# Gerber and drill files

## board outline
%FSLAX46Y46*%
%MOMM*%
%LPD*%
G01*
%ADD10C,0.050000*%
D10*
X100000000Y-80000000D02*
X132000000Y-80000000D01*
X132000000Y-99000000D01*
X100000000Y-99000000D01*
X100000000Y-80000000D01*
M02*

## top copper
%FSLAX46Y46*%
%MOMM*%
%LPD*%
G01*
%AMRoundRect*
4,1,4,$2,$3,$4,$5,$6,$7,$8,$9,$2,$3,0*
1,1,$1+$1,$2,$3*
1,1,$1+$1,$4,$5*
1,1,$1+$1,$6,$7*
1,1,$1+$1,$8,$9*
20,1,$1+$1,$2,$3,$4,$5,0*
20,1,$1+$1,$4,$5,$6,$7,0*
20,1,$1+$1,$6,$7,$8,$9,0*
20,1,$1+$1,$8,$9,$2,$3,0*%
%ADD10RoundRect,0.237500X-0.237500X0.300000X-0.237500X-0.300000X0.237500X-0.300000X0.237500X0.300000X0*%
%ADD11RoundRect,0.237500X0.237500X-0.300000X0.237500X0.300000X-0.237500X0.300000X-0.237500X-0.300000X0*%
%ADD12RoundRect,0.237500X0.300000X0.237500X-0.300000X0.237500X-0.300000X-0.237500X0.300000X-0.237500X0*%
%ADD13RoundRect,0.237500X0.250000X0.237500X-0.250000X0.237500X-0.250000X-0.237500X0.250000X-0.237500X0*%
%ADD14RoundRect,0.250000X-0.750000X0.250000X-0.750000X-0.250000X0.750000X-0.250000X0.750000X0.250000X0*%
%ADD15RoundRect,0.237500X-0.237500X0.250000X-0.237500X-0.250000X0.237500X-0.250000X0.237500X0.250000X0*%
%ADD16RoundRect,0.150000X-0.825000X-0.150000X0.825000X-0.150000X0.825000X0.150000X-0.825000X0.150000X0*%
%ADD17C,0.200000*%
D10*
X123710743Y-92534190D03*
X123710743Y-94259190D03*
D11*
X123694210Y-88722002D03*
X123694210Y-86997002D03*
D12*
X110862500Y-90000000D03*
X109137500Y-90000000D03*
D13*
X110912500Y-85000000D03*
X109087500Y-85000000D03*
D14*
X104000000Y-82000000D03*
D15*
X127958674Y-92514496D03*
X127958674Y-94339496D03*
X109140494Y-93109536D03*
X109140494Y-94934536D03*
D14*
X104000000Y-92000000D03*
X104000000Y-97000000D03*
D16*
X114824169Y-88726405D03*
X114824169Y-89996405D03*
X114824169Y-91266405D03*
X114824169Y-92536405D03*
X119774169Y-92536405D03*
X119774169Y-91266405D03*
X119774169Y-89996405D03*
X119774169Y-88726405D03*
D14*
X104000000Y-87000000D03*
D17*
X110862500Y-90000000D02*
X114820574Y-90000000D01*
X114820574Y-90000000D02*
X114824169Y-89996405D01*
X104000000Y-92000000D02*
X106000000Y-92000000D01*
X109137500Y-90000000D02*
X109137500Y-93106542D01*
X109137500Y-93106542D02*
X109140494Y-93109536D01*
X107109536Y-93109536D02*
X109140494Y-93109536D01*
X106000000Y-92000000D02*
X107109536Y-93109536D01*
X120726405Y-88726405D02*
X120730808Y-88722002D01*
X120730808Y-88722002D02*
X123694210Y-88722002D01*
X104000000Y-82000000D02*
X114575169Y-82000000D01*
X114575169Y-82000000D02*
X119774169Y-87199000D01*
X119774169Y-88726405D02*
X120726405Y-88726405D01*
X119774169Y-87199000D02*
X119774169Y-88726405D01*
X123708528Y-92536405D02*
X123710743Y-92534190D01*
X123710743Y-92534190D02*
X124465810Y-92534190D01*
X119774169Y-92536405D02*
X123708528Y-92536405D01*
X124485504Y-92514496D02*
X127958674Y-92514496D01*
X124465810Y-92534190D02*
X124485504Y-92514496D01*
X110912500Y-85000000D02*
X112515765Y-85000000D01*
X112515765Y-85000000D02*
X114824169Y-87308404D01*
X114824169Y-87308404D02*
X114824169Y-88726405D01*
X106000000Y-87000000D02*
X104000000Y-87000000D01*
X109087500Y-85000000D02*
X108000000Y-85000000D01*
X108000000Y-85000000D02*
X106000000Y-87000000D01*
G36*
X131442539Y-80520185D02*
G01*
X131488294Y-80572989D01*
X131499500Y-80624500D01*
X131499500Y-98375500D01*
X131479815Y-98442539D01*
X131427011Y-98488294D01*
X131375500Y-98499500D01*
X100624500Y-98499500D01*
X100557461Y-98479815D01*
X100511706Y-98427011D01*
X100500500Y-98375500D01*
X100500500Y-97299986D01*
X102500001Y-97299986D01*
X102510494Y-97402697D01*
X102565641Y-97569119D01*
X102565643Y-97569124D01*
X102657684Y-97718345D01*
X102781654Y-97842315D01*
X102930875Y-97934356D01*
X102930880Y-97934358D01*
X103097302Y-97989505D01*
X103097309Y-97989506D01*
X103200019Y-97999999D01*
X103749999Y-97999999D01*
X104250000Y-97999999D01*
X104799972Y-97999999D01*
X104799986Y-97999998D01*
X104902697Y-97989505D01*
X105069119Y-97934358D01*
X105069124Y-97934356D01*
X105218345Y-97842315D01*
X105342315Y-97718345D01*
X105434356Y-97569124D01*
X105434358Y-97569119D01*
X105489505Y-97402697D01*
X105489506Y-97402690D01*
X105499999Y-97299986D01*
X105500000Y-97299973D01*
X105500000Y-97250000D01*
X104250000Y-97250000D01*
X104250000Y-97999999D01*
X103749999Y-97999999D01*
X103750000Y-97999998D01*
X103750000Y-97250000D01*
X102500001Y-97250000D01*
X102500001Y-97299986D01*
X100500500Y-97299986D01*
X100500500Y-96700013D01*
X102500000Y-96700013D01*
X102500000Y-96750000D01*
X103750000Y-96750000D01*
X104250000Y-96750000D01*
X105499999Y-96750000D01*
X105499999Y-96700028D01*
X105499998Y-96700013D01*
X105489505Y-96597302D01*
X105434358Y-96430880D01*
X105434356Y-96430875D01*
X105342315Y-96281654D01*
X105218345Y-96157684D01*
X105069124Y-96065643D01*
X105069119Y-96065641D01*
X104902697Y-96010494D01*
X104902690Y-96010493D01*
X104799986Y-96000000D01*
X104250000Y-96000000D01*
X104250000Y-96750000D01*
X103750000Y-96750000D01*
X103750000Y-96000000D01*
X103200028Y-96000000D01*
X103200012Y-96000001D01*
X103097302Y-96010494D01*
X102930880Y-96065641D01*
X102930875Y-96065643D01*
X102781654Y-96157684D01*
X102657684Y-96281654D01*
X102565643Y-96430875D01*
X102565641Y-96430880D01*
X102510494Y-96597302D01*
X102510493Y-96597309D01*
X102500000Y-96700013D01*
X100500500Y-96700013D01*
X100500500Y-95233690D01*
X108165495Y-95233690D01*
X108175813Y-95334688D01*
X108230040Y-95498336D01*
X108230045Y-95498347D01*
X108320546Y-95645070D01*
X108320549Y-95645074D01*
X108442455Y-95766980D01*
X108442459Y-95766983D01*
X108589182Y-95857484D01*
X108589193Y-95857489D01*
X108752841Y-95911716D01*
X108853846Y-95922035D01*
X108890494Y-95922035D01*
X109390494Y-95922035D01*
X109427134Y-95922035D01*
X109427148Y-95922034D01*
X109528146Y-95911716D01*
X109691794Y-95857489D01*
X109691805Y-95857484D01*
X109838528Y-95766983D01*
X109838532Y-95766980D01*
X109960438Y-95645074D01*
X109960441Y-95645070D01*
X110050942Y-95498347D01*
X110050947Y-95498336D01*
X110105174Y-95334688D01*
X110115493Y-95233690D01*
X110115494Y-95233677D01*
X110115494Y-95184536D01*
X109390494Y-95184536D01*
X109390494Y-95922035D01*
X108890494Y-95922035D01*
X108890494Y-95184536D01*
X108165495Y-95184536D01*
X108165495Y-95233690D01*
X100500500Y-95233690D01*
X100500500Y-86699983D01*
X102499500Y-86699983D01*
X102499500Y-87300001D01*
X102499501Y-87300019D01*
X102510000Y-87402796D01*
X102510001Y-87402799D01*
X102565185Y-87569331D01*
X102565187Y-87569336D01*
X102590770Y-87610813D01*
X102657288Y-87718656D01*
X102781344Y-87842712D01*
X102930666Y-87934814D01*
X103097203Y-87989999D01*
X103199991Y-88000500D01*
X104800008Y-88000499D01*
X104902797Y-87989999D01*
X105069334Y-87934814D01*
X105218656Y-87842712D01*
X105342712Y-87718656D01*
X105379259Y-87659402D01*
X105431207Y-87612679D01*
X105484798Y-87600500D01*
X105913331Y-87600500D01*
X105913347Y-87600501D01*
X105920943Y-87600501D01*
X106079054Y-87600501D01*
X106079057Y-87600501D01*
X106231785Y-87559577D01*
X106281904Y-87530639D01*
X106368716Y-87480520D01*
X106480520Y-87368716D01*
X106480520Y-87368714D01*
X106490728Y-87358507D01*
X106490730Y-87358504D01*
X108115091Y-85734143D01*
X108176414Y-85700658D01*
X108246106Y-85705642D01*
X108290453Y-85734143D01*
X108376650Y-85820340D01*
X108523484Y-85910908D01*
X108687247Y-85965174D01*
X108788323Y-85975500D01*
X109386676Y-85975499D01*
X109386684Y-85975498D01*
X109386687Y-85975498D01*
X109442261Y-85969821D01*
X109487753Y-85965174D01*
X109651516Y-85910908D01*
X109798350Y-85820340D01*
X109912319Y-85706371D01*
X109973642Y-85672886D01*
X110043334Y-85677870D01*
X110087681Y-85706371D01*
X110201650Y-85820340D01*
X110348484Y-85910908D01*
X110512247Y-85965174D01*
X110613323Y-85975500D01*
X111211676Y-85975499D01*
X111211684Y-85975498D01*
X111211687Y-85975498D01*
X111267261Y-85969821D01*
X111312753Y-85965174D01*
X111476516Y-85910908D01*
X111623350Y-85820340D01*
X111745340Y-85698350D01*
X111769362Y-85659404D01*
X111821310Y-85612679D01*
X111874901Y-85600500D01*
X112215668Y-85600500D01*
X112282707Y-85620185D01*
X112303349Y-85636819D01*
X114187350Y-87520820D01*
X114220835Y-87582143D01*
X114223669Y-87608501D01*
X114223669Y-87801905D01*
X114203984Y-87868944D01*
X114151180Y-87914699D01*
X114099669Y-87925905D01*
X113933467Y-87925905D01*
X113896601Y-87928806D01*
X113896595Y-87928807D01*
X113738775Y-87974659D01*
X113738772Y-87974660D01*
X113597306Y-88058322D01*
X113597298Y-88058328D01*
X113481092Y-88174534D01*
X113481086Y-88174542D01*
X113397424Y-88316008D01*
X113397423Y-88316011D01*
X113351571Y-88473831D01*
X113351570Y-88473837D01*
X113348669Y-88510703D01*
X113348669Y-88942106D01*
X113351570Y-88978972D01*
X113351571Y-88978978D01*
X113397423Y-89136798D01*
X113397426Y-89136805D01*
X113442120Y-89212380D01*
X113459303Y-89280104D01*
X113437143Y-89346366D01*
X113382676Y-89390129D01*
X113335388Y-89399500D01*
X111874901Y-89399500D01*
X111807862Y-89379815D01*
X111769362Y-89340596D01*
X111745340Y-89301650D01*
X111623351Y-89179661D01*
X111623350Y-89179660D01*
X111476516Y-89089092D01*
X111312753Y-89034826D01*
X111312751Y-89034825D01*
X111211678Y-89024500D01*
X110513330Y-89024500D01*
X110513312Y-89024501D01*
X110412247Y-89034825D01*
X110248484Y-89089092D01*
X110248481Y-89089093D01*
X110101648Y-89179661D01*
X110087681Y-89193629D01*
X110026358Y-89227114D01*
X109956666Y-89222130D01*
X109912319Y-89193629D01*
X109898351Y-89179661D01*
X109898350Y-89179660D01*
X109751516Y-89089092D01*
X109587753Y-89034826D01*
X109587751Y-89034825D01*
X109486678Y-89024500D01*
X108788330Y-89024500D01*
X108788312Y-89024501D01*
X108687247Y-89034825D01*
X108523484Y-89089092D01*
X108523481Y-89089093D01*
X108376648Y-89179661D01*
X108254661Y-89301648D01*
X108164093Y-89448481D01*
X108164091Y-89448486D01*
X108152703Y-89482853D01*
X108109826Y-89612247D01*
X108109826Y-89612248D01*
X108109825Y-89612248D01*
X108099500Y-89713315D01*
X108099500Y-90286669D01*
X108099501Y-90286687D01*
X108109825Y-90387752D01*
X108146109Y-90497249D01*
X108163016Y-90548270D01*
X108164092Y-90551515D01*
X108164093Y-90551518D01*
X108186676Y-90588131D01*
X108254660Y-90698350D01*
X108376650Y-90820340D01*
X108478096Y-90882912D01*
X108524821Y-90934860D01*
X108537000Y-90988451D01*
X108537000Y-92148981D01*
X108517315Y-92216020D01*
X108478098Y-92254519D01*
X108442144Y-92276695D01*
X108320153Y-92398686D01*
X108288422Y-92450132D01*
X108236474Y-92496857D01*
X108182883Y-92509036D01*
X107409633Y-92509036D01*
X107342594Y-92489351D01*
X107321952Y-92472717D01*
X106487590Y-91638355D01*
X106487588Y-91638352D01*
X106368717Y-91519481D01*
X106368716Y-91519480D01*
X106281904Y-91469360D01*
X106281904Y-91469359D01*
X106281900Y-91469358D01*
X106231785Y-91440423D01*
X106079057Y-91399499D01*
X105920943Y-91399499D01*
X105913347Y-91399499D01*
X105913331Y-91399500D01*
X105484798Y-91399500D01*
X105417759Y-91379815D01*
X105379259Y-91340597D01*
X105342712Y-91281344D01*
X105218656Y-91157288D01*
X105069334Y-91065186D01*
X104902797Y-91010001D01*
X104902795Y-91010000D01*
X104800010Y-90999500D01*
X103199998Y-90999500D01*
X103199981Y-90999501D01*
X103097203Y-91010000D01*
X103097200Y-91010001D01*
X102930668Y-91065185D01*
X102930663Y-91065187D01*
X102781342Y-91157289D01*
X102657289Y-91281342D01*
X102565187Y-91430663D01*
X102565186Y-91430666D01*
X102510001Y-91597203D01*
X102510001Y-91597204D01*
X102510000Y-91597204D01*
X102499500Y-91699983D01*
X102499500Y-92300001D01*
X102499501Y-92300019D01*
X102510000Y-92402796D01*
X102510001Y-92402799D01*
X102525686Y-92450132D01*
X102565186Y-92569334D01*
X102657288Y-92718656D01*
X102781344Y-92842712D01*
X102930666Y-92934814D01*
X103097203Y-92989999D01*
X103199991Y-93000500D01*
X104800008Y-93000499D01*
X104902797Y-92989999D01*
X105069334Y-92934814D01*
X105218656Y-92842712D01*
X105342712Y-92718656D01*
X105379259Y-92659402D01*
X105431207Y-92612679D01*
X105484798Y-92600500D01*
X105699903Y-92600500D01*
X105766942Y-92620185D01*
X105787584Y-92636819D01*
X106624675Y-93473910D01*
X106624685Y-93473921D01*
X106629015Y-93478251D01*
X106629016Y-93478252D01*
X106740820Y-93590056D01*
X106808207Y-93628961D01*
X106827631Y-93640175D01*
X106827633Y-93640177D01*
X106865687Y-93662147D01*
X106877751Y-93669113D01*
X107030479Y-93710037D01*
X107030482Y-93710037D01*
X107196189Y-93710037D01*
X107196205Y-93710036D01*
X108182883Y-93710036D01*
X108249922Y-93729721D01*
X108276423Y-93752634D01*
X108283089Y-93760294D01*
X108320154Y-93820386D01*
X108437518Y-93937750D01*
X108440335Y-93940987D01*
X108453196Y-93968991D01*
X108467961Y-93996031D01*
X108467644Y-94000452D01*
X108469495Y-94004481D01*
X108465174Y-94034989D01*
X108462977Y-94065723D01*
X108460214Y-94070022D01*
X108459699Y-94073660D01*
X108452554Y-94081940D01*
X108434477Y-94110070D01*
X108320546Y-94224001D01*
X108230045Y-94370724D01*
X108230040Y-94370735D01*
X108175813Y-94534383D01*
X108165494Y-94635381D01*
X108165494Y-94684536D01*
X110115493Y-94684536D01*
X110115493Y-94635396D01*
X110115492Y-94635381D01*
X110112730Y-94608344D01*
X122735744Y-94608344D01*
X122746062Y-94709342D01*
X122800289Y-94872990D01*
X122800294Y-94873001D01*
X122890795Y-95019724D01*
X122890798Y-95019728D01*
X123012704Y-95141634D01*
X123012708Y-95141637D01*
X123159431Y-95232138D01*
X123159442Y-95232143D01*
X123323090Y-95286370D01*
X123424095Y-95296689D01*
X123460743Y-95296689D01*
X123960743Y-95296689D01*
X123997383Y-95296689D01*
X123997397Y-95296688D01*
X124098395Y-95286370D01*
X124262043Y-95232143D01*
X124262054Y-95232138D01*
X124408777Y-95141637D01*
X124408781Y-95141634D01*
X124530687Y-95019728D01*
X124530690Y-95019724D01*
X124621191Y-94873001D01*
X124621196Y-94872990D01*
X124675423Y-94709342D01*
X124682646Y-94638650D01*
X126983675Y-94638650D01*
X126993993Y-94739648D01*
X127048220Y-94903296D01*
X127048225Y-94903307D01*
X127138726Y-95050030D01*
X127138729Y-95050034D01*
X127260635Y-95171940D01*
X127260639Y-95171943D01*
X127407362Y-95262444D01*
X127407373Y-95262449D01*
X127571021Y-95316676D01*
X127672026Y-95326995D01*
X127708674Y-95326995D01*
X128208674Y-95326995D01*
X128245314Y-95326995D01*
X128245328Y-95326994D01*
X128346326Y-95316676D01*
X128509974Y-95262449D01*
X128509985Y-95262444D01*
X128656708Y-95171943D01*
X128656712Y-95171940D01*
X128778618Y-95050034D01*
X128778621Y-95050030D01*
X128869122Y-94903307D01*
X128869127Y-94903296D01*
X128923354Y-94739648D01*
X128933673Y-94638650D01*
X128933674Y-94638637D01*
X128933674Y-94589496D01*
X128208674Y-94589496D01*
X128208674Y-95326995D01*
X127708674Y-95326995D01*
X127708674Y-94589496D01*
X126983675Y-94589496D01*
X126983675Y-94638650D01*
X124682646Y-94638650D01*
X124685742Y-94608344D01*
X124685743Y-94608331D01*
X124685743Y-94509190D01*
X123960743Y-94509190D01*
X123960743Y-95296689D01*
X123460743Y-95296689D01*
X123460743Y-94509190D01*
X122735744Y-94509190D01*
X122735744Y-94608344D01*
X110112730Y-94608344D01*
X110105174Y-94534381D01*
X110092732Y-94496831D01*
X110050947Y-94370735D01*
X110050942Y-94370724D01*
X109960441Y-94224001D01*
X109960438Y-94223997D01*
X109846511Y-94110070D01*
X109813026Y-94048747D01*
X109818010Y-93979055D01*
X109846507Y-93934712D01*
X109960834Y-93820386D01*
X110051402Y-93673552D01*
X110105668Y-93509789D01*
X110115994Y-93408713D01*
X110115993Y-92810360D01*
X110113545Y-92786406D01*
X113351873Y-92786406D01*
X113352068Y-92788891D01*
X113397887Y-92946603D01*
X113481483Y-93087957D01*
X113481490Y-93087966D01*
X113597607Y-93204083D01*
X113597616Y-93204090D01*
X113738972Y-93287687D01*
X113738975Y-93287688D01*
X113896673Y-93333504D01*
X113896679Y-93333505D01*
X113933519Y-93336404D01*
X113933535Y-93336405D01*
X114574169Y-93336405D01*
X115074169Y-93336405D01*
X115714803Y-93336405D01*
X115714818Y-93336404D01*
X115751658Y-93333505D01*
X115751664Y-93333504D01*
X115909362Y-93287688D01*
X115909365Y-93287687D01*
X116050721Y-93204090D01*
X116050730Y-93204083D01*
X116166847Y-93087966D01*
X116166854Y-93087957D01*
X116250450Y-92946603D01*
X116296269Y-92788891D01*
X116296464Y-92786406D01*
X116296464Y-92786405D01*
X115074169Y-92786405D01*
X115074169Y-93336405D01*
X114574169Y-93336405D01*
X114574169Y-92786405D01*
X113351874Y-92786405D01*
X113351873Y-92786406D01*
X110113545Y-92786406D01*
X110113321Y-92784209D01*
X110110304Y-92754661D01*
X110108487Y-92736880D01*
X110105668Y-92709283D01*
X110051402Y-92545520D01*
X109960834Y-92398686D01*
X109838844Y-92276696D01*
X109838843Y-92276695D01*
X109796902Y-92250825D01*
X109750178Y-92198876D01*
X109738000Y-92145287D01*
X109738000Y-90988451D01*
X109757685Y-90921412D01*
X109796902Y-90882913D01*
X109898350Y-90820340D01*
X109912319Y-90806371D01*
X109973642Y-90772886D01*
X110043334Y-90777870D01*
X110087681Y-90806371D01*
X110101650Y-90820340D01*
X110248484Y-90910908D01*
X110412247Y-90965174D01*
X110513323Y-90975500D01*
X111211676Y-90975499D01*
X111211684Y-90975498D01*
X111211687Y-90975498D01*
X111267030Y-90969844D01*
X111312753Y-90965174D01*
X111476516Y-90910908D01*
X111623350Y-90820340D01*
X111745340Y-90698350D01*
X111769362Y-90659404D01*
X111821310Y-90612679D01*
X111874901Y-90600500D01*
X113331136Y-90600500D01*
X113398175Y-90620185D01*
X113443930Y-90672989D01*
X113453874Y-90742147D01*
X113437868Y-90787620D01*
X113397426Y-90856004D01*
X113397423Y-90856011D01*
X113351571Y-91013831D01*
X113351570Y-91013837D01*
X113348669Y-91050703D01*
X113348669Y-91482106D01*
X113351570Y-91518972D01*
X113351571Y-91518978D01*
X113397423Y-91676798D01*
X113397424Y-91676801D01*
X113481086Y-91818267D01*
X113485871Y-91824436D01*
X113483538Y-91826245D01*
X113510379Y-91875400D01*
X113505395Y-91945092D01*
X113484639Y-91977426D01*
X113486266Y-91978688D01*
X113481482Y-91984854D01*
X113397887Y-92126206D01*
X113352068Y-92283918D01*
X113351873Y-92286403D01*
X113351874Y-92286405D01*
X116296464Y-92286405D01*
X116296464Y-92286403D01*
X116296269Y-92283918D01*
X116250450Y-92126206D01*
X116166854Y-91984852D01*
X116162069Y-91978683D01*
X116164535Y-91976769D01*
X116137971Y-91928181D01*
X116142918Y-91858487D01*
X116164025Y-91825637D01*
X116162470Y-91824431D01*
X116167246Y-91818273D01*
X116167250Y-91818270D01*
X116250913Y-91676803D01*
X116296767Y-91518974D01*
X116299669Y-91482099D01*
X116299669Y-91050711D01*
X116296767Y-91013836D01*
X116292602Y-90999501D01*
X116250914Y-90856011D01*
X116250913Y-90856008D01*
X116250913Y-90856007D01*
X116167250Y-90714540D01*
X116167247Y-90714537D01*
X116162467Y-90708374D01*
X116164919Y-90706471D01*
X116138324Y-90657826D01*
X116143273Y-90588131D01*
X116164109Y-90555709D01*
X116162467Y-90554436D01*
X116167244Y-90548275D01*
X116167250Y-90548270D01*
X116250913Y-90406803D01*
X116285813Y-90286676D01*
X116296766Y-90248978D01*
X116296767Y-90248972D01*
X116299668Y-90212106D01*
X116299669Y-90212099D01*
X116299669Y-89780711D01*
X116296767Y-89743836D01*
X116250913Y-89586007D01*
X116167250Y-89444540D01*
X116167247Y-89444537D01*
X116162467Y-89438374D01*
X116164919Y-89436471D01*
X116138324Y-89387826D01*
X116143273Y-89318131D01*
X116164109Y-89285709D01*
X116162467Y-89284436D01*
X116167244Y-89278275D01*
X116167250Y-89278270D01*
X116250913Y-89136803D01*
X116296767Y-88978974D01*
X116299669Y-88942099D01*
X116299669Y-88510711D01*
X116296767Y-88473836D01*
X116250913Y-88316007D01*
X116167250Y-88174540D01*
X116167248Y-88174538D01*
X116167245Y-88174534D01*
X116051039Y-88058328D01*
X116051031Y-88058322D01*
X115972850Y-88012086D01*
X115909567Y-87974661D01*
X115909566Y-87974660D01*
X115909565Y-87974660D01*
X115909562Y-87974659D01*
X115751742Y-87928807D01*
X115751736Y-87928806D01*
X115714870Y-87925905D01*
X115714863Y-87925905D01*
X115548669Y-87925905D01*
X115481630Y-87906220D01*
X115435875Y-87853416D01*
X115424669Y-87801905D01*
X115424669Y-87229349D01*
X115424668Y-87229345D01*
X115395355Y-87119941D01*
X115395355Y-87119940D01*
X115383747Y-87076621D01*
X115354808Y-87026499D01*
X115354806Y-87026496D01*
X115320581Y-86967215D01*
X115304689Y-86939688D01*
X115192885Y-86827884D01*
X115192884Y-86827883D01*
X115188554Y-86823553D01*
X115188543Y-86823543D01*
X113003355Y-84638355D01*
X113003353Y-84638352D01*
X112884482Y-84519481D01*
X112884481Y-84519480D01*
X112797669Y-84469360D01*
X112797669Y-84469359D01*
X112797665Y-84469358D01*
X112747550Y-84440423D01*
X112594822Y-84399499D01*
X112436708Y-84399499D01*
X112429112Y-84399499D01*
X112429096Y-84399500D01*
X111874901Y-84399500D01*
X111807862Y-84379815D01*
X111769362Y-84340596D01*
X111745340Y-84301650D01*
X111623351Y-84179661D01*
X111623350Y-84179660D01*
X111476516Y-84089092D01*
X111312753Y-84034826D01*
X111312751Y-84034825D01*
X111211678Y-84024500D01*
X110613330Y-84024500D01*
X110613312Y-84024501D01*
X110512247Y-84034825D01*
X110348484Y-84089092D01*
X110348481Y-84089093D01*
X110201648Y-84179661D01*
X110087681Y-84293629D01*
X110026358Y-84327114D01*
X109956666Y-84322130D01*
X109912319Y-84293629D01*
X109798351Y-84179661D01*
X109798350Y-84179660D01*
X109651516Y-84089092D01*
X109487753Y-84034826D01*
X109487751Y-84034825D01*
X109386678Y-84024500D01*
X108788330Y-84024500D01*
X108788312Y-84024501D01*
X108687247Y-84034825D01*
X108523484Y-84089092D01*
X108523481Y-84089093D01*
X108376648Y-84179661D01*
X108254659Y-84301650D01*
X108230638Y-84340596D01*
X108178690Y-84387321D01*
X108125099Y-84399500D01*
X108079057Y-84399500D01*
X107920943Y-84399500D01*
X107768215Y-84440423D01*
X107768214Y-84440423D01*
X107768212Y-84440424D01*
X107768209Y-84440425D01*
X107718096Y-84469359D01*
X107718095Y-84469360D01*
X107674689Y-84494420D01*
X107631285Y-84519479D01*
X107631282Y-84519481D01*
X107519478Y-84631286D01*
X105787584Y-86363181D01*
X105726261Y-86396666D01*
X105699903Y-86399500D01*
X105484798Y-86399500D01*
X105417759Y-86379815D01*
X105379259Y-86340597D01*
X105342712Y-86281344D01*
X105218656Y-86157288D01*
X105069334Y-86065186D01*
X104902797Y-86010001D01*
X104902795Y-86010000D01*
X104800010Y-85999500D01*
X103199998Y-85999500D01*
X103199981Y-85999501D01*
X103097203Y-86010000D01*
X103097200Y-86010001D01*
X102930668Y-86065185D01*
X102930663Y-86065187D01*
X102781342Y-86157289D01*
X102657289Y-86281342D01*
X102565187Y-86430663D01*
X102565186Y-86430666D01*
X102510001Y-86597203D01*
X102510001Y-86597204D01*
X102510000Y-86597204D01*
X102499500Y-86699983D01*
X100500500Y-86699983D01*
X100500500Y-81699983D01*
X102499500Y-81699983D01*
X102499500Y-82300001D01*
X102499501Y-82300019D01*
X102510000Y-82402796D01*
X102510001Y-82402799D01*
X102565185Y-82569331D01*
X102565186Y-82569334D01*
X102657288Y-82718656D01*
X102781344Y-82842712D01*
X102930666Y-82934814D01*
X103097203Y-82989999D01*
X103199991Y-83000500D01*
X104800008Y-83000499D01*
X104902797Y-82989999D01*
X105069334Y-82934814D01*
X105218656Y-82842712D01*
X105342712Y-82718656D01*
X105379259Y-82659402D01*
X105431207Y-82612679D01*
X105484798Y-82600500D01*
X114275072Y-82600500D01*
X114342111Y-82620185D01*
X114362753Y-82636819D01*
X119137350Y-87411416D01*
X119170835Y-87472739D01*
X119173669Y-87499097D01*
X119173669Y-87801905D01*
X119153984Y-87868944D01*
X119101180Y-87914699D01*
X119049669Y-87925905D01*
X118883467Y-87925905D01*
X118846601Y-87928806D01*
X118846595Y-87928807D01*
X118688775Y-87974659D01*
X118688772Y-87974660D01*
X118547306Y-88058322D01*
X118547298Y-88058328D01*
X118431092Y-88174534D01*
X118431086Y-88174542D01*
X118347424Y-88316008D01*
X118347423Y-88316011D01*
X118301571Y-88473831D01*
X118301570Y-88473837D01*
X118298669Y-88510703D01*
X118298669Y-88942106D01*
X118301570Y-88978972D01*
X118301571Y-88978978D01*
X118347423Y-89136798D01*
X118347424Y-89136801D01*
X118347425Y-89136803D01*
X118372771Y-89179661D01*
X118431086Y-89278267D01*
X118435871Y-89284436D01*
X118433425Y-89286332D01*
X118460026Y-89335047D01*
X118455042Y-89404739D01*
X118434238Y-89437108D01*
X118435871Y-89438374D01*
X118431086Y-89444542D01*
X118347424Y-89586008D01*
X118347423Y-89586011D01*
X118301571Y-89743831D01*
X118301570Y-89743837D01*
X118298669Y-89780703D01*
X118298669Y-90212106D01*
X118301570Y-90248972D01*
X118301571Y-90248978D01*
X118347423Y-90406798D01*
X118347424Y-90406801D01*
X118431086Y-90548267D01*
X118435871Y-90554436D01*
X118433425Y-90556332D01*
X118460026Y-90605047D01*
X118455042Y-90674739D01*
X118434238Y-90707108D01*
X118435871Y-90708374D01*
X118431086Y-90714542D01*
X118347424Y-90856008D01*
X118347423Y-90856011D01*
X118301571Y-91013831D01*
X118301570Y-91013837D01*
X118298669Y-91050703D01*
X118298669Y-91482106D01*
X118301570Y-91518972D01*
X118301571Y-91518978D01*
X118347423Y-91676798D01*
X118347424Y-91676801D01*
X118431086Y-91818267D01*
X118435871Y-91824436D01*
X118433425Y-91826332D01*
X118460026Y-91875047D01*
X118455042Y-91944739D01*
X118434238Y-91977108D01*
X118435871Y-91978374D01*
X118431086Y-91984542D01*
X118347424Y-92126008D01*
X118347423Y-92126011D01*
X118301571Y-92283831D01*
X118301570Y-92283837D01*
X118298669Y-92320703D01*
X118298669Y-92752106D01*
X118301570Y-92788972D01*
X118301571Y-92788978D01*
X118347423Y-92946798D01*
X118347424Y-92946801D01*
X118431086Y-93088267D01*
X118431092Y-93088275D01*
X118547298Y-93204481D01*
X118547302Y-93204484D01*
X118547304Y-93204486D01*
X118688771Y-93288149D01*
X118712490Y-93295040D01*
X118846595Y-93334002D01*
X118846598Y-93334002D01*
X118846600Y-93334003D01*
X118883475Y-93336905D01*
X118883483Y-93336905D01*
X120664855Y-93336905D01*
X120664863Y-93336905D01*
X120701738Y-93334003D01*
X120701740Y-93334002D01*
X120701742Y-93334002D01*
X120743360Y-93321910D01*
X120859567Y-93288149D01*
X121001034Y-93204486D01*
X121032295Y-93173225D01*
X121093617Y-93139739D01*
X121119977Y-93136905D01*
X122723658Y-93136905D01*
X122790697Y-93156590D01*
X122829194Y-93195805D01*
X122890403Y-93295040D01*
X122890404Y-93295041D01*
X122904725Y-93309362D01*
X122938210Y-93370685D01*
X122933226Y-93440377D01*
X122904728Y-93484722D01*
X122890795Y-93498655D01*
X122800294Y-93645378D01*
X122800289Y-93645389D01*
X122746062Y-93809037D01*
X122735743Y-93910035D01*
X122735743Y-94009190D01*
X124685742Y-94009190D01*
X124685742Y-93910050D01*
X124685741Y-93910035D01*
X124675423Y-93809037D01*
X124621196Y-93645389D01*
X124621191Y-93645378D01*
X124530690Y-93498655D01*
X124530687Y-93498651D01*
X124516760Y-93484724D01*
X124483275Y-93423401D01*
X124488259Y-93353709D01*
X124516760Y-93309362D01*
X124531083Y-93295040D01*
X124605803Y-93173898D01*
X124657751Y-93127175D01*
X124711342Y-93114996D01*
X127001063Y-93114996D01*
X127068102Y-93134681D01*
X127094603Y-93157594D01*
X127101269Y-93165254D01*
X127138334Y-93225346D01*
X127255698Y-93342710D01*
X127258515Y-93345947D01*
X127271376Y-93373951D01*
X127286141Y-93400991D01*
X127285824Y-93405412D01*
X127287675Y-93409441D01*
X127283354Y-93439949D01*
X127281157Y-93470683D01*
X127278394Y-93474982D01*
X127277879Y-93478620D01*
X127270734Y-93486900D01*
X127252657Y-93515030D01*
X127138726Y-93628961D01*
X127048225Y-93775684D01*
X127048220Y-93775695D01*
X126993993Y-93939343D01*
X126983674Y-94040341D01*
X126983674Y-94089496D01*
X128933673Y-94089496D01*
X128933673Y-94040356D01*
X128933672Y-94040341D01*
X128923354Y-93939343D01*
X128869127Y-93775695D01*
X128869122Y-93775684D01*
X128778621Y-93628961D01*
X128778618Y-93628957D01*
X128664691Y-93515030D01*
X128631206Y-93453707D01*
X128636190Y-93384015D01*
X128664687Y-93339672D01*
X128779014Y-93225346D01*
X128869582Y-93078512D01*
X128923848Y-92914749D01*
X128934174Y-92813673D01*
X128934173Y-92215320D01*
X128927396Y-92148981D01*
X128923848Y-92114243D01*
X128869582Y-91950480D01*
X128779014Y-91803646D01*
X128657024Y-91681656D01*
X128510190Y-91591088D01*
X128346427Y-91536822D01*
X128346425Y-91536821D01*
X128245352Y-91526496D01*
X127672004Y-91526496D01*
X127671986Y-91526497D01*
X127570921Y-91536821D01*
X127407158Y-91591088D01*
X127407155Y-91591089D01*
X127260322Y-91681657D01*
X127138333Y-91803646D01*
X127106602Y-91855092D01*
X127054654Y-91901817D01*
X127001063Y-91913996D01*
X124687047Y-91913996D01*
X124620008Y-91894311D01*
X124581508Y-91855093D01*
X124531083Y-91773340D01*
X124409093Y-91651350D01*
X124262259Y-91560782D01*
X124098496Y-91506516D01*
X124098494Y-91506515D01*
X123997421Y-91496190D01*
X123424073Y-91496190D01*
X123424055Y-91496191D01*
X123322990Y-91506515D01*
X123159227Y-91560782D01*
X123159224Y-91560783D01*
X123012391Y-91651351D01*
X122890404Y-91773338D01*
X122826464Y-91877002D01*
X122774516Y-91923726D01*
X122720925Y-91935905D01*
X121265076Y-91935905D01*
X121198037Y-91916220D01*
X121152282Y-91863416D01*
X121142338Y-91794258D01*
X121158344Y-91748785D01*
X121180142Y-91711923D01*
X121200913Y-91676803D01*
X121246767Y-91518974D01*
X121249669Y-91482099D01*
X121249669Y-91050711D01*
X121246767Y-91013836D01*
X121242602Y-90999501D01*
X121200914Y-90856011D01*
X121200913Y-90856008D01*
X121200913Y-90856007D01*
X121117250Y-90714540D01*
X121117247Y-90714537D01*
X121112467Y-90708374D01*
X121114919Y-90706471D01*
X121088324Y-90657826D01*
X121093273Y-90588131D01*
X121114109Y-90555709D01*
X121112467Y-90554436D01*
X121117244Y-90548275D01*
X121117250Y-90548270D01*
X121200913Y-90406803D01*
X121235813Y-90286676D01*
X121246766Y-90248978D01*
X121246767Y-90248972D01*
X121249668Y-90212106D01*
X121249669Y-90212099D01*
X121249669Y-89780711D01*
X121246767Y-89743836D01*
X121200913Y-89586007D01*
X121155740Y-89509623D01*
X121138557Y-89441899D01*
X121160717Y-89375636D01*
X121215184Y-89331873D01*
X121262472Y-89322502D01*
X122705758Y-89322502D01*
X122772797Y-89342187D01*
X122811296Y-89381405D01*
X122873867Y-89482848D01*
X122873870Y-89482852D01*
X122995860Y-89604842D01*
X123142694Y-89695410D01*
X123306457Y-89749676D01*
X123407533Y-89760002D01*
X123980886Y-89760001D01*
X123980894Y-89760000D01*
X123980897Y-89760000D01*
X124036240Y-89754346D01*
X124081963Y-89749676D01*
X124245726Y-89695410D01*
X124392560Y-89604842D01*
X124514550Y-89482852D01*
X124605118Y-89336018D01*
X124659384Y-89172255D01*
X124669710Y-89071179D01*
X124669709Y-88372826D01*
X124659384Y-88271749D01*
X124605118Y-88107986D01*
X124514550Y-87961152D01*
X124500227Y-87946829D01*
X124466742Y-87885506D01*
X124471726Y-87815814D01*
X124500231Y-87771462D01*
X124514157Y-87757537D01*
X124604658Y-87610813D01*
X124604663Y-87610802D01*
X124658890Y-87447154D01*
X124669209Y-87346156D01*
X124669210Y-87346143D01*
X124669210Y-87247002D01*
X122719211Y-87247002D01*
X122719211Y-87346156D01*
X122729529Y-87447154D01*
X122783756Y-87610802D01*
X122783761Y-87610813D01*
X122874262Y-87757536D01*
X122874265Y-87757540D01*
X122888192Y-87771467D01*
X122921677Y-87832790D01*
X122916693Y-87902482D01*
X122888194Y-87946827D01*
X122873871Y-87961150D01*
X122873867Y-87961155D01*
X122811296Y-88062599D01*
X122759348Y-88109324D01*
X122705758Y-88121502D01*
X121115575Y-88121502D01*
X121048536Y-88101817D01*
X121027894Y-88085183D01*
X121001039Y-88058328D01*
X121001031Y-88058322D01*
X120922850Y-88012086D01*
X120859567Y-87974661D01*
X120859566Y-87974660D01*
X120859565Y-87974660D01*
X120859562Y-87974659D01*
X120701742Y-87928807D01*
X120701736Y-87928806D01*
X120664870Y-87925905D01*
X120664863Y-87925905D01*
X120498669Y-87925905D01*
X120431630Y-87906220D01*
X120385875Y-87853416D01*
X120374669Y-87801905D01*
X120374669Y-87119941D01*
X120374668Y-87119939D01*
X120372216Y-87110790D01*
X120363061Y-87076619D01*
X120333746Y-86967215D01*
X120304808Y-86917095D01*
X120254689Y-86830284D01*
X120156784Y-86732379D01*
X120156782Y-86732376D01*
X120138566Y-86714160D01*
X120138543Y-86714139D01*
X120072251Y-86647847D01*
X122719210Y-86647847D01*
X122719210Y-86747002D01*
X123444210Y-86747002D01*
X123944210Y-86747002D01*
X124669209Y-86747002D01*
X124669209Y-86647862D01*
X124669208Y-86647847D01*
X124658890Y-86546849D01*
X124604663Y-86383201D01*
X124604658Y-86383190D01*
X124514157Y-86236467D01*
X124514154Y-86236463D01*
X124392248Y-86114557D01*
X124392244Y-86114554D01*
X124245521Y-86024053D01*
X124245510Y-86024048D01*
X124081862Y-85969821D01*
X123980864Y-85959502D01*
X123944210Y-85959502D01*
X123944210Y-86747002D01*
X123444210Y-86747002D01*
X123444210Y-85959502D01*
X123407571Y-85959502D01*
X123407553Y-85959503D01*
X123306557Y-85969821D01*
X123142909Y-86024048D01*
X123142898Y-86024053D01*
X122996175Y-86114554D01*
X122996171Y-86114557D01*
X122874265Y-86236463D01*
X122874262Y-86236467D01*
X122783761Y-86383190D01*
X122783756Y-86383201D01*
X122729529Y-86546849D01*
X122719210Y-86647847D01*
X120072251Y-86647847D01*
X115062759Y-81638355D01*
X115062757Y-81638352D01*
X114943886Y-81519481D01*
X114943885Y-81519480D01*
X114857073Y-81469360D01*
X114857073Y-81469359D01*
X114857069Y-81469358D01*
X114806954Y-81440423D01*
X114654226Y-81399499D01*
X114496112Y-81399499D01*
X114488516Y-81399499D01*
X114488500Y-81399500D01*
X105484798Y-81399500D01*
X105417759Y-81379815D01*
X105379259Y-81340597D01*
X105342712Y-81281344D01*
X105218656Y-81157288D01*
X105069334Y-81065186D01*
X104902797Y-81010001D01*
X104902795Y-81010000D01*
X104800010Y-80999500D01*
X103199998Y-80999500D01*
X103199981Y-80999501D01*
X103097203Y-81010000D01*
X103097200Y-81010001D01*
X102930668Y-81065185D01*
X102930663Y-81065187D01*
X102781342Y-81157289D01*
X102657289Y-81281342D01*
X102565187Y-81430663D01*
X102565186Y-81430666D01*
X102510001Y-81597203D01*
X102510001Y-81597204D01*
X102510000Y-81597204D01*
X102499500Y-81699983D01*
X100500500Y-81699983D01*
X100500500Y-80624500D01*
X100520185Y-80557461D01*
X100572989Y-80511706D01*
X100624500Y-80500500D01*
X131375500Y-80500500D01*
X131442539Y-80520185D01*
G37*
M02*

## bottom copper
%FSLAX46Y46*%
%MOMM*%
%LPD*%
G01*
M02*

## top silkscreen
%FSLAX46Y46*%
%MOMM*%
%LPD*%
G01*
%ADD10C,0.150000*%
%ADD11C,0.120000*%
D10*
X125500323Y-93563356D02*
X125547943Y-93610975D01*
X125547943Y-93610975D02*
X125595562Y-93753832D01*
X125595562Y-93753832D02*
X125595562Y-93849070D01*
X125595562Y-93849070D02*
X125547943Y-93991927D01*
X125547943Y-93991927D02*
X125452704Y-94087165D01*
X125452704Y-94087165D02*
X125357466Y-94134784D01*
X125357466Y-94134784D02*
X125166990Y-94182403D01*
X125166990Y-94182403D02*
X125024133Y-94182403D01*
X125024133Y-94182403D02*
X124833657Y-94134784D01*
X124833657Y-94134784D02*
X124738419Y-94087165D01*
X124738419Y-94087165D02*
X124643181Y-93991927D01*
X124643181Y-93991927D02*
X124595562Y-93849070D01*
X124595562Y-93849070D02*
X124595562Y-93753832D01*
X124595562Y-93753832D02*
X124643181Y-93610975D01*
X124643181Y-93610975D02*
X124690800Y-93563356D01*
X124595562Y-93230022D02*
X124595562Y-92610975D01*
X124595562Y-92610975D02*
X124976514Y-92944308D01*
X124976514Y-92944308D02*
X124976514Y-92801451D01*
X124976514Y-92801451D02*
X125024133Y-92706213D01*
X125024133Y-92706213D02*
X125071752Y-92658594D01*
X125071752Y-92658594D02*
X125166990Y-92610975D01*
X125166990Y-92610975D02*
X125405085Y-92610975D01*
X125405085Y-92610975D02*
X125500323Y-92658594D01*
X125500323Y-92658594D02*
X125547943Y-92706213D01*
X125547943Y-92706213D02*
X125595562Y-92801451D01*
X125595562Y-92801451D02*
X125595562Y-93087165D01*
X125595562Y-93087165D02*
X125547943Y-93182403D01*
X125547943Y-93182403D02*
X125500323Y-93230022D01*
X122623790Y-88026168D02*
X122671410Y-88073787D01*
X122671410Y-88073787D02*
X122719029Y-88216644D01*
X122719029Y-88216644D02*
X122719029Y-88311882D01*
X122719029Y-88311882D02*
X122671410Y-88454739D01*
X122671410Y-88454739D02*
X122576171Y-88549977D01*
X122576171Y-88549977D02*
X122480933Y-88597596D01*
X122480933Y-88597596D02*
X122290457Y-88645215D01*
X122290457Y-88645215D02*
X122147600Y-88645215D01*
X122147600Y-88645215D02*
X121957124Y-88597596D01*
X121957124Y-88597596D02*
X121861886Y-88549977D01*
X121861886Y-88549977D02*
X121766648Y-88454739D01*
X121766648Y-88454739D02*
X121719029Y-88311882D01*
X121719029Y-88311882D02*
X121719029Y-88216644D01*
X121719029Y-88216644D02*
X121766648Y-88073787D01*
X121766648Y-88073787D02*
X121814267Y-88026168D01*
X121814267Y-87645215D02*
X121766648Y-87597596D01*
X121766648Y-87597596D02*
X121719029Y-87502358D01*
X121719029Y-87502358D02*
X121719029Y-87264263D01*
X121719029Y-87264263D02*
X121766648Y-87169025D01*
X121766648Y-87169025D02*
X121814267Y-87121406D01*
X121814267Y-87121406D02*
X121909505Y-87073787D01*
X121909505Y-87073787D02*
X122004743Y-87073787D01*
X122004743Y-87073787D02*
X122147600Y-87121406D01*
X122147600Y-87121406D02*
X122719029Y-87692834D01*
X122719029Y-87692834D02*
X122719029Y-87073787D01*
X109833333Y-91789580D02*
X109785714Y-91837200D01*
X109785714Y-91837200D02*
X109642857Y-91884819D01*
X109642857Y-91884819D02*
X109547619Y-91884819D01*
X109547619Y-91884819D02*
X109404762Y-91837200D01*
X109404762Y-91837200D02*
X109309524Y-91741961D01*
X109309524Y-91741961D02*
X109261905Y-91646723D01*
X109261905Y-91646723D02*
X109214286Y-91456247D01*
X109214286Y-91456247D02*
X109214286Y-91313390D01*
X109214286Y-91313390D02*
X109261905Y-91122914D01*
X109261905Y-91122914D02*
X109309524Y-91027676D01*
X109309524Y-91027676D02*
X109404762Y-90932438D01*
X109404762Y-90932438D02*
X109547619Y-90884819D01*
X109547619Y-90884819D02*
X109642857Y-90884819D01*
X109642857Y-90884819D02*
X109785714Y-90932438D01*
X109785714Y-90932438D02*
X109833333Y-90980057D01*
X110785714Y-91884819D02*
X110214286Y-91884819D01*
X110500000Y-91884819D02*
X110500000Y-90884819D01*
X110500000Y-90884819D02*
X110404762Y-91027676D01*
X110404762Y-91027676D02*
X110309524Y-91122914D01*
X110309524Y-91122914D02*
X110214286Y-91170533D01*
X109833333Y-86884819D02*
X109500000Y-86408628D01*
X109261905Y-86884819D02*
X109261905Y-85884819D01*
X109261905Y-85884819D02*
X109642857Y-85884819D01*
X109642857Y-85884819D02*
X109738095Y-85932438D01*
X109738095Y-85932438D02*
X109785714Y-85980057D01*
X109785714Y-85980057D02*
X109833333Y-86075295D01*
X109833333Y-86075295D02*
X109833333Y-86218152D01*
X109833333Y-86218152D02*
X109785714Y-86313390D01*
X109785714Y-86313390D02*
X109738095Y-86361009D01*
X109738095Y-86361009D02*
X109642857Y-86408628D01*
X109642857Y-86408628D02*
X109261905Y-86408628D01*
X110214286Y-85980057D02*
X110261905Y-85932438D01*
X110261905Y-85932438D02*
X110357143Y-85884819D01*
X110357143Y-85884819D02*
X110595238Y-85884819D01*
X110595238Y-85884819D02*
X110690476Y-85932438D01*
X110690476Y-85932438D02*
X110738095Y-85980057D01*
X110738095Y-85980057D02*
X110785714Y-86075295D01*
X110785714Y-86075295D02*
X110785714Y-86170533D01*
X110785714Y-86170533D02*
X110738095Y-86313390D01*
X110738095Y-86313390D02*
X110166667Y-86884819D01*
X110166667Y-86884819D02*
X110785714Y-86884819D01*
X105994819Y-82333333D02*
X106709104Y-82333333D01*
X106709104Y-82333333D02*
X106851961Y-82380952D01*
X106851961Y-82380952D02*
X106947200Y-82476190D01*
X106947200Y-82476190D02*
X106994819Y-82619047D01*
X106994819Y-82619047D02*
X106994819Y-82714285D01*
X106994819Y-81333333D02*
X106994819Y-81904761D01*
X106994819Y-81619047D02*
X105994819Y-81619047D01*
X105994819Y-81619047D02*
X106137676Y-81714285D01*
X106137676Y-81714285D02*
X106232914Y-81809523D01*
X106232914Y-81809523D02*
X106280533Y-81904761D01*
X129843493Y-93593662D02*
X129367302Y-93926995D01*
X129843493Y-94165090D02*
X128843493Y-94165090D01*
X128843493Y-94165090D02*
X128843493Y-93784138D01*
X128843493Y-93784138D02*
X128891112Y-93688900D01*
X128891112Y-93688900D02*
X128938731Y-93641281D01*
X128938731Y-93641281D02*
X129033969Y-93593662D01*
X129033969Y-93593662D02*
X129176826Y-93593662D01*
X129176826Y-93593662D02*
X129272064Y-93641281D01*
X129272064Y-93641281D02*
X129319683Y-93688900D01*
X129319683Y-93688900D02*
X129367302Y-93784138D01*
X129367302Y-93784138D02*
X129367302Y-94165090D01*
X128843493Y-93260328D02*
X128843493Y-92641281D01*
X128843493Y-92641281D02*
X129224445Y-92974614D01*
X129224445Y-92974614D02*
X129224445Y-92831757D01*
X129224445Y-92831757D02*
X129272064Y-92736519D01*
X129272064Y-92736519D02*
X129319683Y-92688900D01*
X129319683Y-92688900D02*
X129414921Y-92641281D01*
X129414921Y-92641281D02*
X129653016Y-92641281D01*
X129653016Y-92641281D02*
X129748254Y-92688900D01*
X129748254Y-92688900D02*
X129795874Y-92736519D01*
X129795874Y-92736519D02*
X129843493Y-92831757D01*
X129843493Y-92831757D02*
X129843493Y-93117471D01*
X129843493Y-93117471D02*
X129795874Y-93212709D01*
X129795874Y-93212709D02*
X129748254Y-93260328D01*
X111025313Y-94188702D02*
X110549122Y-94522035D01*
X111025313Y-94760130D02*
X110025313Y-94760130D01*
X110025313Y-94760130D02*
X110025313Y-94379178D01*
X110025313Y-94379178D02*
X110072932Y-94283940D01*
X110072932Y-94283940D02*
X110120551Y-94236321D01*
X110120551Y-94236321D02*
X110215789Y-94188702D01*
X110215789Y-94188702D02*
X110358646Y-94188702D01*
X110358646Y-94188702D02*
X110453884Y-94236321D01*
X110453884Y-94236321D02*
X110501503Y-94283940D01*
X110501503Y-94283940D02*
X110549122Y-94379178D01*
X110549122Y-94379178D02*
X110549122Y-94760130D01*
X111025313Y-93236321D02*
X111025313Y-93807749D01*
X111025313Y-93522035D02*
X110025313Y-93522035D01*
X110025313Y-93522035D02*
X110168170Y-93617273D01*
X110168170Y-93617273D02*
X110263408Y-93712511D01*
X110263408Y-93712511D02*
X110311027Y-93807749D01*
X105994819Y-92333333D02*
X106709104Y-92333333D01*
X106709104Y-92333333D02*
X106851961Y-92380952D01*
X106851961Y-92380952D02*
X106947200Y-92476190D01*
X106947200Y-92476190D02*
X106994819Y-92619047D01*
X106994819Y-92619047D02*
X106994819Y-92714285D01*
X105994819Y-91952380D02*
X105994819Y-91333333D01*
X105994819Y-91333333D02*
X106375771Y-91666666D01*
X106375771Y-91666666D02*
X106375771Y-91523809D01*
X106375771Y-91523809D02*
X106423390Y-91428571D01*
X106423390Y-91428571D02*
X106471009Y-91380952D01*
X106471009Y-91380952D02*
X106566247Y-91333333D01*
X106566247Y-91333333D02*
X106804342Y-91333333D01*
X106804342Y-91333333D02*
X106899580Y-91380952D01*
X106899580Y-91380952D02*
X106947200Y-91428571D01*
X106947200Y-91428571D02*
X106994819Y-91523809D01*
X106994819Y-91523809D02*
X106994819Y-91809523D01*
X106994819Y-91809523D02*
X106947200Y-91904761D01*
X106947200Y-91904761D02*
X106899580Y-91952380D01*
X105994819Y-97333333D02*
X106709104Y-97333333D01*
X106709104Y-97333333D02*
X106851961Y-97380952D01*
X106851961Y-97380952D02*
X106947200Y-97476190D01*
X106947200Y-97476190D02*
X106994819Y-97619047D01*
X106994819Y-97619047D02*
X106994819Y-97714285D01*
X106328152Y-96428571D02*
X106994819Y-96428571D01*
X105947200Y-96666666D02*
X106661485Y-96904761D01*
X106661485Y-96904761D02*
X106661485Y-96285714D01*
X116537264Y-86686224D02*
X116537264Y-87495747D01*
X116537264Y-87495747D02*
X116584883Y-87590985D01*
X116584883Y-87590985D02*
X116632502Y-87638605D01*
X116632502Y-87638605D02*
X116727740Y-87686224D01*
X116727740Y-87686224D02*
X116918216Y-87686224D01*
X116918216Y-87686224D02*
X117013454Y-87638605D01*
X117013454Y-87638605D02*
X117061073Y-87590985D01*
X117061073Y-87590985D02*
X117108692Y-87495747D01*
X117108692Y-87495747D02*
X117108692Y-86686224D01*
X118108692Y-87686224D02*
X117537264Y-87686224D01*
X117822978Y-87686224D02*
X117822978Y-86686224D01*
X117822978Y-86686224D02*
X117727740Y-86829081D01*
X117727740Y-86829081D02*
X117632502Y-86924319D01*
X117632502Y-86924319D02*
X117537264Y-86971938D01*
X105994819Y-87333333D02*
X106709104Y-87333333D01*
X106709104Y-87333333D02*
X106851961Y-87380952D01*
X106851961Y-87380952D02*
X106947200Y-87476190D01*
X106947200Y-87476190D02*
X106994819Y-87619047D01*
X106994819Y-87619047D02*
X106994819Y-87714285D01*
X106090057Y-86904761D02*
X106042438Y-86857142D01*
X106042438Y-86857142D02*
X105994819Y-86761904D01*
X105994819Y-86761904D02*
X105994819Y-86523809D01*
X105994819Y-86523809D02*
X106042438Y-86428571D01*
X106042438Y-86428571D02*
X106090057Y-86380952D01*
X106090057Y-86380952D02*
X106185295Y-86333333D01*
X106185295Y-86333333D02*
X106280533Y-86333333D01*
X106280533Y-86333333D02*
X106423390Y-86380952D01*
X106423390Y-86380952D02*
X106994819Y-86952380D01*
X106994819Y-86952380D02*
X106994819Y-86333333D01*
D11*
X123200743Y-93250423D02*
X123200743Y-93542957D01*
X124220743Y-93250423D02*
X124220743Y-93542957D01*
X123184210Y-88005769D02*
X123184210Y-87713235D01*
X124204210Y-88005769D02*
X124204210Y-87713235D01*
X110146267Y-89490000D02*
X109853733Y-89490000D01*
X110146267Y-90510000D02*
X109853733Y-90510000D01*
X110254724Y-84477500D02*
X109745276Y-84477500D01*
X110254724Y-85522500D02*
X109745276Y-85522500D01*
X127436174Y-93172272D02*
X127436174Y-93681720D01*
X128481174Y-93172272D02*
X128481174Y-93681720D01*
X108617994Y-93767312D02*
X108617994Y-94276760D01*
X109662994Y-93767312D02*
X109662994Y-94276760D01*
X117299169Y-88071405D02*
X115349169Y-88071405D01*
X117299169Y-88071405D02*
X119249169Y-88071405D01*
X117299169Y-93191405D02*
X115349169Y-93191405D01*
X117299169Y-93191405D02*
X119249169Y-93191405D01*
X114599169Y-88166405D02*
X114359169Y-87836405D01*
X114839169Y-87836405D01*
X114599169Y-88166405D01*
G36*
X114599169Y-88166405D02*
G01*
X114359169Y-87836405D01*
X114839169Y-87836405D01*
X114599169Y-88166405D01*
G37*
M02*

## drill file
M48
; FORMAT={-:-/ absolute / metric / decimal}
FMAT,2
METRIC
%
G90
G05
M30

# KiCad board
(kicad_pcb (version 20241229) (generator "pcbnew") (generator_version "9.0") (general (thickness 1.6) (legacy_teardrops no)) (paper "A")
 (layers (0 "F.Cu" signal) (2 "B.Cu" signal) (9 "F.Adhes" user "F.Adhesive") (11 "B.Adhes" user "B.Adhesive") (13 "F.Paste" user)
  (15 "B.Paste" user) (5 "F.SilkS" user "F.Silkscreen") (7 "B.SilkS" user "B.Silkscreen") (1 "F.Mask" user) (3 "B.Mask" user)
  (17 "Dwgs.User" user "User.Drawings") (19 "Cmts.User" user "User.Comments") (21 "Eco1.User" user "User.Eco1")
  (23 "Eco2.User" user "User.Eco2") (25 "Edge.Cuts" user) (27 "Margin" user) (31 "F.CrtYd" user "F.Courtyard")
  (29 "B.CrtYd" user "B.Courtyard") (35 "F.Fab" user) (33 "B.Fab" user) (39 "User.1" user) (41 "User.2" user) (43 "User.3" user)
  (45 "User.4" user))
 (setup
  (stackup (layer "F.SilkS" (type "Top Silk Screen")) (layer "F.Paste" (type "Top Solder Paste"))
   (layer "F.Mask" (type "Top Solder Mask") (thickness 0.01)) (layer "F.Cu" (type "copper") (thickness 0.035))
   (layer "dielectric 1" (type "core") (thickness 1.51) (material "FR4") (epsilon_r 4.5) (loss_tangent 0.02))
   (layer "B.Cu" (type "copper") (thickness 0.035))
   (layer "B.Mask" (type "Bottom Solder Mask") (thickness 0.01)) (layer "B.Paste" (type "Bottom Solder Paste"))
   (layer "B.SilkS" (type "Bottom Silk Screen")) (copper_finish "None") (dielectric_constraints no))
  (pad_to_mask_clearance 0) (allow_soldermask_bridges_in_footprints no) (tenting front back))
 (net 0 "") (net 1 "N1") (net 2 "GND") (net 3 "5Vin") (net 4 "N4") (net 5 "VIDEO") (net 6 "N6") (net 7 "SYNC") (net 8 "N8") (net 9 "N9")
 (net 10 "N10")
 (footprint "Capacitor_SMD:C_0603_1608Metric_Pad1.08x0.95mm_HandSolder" (layer "F.Cu") (at 123.710743 93.39669 -90)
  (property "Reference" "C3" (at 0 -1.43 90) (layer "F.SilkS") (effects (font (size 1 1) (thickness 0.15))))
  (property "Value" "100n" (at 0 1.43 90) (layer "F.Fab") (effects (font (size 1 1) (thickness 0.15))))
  (fp_line (start -0.146267 0.51) (end 0.146267 0.51) (stroke (width 0.12) (type solid)) (layer "F.SilkS"))
  (fp_line (start -0.146267 -0.51) (end 0.146267 -0.51) (stroke (width 0.12) (type solid)) (layer "F.SilkS"))
  (pad "1" smd roundrect (at -0.8625 0 270) (size 1.075 0.95) (layers "F.Cu" "F.Mask" "F.Paste") (roundrect_rratio 0.25) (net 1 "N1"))
  (pad "2" smd roundrect (at 0.8625 0 270) (size 1.075 0.95) (layers "F.Cu" "F.Mask" "F.Paste") (roundrect_rratio 0.25) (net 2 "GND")))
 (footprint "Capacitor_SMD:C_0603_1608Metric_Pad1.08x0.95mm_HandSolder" (layer "F.Cu") (at 123.69421 87.859502 90)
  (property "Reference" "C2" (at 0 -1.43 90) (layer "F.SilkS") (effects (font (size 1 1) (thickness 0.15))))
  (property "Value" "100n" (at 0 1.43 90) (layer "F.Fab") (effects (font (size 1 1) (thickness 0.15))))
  (fp_line (start -0.146267 -0.51) (end 0.146267 -0.51) (stroke (width 0.12) (type solid)) (layer "F.SilkS"))
  (fp_line (start -0.146267 0.51) (end 0.146267 0.51) (stroke (width 0.12) (type solid)) (layer "F.SilkS"))
  (pad "1" smd roundrect (at -0.8625 0 90) (size 1.075 0.95) (layers "F.Cu" "F.Mask" "F.Paste") (roundrect_rratio 0.25) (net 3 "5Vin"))
  (pad "2" smd roundrect (at 0.8625 0 90) (size 1.075 0.95) (layers "F.Cu" "F.Mask" "F.Paste") (roundrect_rratio 0.25) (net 2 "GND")))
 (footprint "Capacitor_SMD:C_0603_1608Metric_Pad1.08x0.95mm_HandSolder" (layer "F.Cu") (at 110 90 180)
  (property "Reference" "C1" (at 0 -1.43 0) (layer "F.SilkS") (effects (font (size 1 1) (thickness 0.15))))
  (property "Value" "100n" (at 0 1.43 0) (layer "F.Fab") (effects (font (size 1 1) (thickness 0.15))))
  (fp_line (start -0.146267 0.51) (end 0.146267 0.51) (stroke (width 0.12) (type solid)) (layer "F.SilkS"))
  (fp_line (start -0.146267 -0.51) (end 0.146267 -0.51) (stroke (width 0.12) (type solid)) (layer "F.SilkS"))
  (pad "1" smd roundrect (at -0.8625 0 180) (size 1.075 0.95) (layers "F.Cu" "F.Mask" "F.Paste") (roundrect_rratio 0.25) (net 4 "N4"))
  (pad "2" smd roundrect (at 0.8625 0 180) (size 1.075 0.95) (layers "F.Cu" "F.Mask" "F.Paste") (roundrect_rratio 0.25) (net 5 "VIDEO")))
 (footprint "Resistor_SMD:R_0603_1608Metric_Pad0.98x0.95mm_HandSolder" (layer "F.Cu") (at 110 85 180)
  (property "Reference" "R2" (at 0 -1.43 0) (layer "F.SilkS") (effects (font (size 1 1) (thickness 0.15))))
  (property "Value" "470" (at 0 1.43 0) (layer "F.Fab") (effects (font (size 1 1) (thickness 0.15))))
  (fp_line (start -0.254724 0.5225) (end 0.254724 0.5225) (stroke (width 0.12) (type solid)) (layer "F.SilkS"))
  (fp_line (start -0.254724 -0.5225) (end 0.254724 -0.5225) (stroke (width 0.12) (type solid)) (layer "F.SilkS"))
  (pad "1" smd roundrect (at -0.9125 0 180) (size 0.975 0.95) (layers "F.Cu" "F.Mask" "F.Paste") (roundrect_rratio 0.25) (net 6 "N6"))
  (pad "2" smd roundrect (at 0.9125 0 180) (size 0.975 0.95) (layers "F.Cu" "F.Mask" "F.Paste") (roundrect_rratio 0.25) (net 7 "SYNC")))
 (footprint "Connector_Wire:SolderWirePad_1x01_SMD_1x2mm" (layer "F.Cu") (at 104 82 -90)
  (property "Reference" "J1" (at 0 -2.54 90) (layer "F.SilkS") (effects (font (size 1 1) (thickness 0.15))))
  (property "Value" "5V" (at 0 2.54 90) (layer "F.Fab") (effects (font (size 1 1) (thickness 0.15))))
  (pad "1" smd roundrect (at 0 0 270) (size 1 2) (layers "F.Cu" "F.Mask" "F.Paste") (roundrect_rratio 0.25) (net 3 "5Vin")))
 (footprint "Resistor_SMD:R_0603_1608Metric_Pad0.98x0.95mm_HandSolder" (layer "F.Cu") (at 127.958674 93.426996 -90)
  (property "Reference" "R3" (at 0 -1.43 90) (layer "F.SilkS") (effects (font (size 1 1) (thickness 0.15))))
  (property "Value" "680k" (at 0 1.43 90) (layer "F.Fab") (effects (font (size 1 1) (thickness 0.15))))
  (fp_line (start -0.254724 0.5225) (end 0.254724 0.5225) (stroke (width 0.12) (type solid)) (layer "F.SilkS"))
  (fp_line (start -0.254724 -0.5225) (end 0.254724 -0.5225) (stroke (width 0.12) (type solid)) (layer "F.SilkS"))
  (pad "1" smd roundrect (at -0.9125 0 270) (size 0.975 0.95) (layers "F.Cu" "F.Mask" "F.Paste") (roundrect_rratio 0.25) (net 1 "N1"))
  (pad "2" smd roundrect (at 0.9125 0 270) (size 0.975 0.95) (layers "F.Cu" "F.Mask" "F.Paste") (roundrect_rratio 0.25) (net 2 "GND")))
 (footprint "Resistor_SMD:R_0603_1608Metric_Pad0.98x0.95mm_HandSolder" (layer "F.Cu") (at 109.140494 94.022036 -90)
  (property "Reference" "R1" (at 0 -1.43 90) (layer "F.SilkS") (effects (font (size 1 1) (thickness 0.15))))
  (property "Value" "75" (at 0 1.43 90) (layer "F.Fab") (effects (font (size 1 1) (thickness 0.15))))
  (fp_line (start -0.254724 0.5225) (end 0.254724 0.5225) (stroke (width 0.12) (type solid)) (layer "F.SilkS"))
  (fp_line (start -0.254724 -0.5225) (end 0.254724 -0.5225) (stroke (width 0.12) (type solid)) (layer "F.SilkS"))
  (pad "1" smd roundrect (at -0.9125 0 270) (size 0.975 0.95) (layers "F.Cu" "F.Mask" "F.Paste") (roundrect_rratio 0.25) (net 5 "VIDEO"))
  (pad "2" smd roundrect (at 0.9125 0 270) (size 0.975 0.95) (layers "F.Cu" "F.Mask" "F.Paste") (roundrect_rratio 0.25) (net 2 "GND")))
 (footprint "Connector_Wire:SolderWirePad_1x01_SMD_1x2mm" (layer "F.Cu") (at 104 92 -90)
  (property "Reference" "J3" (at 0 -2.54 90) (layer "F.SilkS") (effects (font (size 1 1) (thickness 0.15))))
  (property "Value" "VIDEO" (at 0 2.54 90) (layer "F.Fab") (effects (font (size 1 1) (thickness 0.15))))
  (pad "1" smd roundrect (at 0 0 270) (size 1 2) (layers "F.Cu" "F.Mask" "F.Paste") (roundrect_rratio 0.25) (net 5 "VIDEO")))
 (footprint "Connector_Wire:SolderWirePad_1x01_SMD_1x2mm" (layer "F.Cu") (at 104 97 -90)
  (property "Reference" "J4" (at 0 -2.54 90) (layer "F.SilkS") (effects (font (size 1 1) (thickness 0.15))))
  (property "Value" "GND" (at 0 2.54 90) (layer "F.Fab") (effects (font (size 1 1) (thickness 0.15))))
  (pad "1" smd roundrect (at 0 0 270) (size 1 2) (layers "F.Cu" "F.Mask" "F.Paste") (roundrect_rratio 0.25) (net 2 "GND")))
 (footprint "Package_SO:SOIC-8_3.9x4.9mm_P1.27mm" (layer "F.Cu") (at 117.299169 90.631405)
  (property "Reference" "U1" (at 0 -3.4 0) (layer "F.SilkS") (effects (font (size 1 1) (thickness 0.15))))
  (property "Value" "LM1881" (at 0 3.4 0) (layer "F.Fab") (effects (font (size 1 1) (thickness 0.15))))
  (fp_line (start 0 -2.56) (end -1.95 -2.56) (stroke (width 0.12) (type solid)) (layer "F.SilkS"))
  (fp_line (start 0 -2.56) (end 1.95 -2.56) (stroke (width 0.12) (type solid)) (layer "F.SilkS"))
  (fp_line (start 0 2.56) (end -1.95 2.56) (stroke (width 0.12) (type solid)) (layer "F.SilkS"))
  (fp_line (start 0 2.56) (end 1.95 2.56) (stroke (width 0.12) (type solid)) (layer "F.SilkS"))
  (fp_poly
   (pts (xy -2.7 -2.465) (xy -2.94 -2.795) (xy -2.46 -2.795) (xy -2.7 -2.465)) (stroke (width 0.12) (type solid)) (fill yes)
   (layer "F.SilkS"))
  (pad "1" smd roundrect (at -2.475 -1.905) (size 1.95 0.6) (layers "F.Cu" "F.Mask" "F.Paste") (roundrect_rratio 0.25) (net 6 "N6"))
  (pad "2" smd roundrect (at -2.475 -0.635) (size 1.95 0.6) (layers "F.Cu" "F.Mask" "F.Paste") (roundrect_rratio 0.25) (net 4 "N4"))
  (pad "3" smd roundrect (at -2.475 0.635) (size 1.95 0.6) (layers "F.Cu" "F.Mask" "F.Paste") (roundrect_rratio 0.25) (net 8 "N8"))
  (pad "4" smd roundrect (at -2.475 1.905) (size 1.95 0.6) (layers "F.Cu" "F.Mask" "F.Paste") (roundrect_rratio 0.25) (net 2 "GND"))
  (pad "5" smd roundrect (at 2.475 1.905) (size 1.95 0.6) (layers "F.Cu" "F.Mask" "F.Paste") (roundrect_rratio 0.25) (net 1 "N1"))
  (pad "6" smd roundrect (at 2.475 0.635) (size 1.95 0.6) (layers "F.Cu" "F.Mask" "F.Paste") (roundrect_rratio 0.25) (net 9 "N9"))
  (pad "7" smd roundrect (at 2.475 -0.635) (size 1.95 0.6) (layers "F.Cu" "F.Mask" "F.Paste") (roundrect_rratio 0.25) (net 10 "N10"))
  (pad "8" smd roundrect (at 2.475 -1.905) (size 1.95 0.6) (layers "F.Cu" "F.Mask" "F.Paste") (roundrect_rratio 0.25) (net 3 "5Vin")))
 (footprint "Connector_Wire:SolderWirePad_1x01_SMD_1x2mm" (layer "F.Cu") (at 104 87 -90)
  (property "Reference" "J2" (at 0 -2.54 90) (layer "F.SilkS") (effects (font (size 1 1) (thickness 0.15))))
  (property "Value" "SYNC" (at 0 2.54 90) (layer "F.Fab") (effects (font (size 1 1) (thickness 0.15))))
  (pad "1" smd roundrect (at 0 0 270) (size 1 2) (layers "F.Cu" "F.Mask" "F.Paste") (roundrect_rratio 0.25) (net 7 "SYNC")))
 (gr_rect (start 100 80) (end 132 99) (stroke (width 0.05) (type default)) (fill no) (layer "Edge.Cuts"))
 (segment (start 110.8625 90) (end 114.820574 90) (width 0.2) (layer "F.Cu") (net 4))
 (segment (start 114.820574 90) (end 114.824169 89.996405) (width 0.2) (layer "F.Cu") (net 4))
 (segment (start 104 92) (end 106 92) (width 0.2) (layer "F.Cu") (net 5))
 (segment (start 109.1375 90) (end 109.1375 93.106542) (width 0.2) (layer "F.Cu") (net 5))
 (segment (start 109.1375 93.106542) (end 109.140494 93.109536) (width 0.2) (layer "F.Cu") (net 5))
 (segment (start 107.109536 93.109536) (end 109.140494 93.109536) (width 0.2) (layer "F.Cu") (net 5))
 (segment (start 106 92) (end 107.109536 93.109536) (width 0.2) (layer "F.Cu") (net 5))
 (segment (start 120.726405 88.726405) (end 120.730808 88.722002) (width 0.2) (layer "F.Cu") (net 3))
 (segment (start 120.730808 88.722002) (end 123.69421 88.722002) (width 0.2) (layer "F.Cu") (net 3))
 (segment (start 104 82) (end 114.575169 82) (width 0.2) (layer "F.Cu") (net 3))
 (segment (start 114.575169 82) (end 119.774169 87.199) (width 0.2) (layer "F.Cu") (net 3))
 (segment (start 119.774169 88.726405) (end 120.726405 88.726405) (width 0.2) (layer "F.Cu") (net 3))
 (segment (start 119.774169 87.199) (end 119.774169 88.726405) (width 0.2) (layer "F.Cu") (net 3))
 (segment (start 123.708528 92.536405) (end 123.710743 92.53419) (width 0.2) (layer "F.Cu") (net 1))
 (segment (start 123.710743 92.53419) (end 124.46581 92.53419) (width 0.2) (layer "F.Cu") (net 1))
 (segment (start 119.774169 92.536405) (end 123.708528 92.536405) (width 0.2) (layer "F.Cu") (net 1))
 (segment (start 124.485504 92.514496) (end 127.958674 92.514496) (width 0.2) (layer "F.Cu") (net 1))
 (segment (start 124.46581 92.53419) (end 124.485504 92.514496) (width 0.2) (layer "F.Cu") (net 1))
 (segment (start 110.9125 85) (end 112.515765 85) (width 0.2) (layer "F.Cu") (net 6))
 (segment (start 112.515765 85) (end 114.824169 87.308404) (width 0.2) (layer "F.Cu") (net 6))
 (segment (start 114.824169 87.308404) (end 114.824169 88.726405) (width 0.2) (layer "F.Cu") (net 6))
 (segment (start 106 87) (end 104 87) (width 0.2) (layer "F.Cu") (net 7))
 (segment (start 109.0875 85) (end 108 85) (width 0.2) (layer "F.Cu") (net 7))
 (segment (start 108 85) (end 106 87) (width 0.2) (layer "F.Cu") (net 7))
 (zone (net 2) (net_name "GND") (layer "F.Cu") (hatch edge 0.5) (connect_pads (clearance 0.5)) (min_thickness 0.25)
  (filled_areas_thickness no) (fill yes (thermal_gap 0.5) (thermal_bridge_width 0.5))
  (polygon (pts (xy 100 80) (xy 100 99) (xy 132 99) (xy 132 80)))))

